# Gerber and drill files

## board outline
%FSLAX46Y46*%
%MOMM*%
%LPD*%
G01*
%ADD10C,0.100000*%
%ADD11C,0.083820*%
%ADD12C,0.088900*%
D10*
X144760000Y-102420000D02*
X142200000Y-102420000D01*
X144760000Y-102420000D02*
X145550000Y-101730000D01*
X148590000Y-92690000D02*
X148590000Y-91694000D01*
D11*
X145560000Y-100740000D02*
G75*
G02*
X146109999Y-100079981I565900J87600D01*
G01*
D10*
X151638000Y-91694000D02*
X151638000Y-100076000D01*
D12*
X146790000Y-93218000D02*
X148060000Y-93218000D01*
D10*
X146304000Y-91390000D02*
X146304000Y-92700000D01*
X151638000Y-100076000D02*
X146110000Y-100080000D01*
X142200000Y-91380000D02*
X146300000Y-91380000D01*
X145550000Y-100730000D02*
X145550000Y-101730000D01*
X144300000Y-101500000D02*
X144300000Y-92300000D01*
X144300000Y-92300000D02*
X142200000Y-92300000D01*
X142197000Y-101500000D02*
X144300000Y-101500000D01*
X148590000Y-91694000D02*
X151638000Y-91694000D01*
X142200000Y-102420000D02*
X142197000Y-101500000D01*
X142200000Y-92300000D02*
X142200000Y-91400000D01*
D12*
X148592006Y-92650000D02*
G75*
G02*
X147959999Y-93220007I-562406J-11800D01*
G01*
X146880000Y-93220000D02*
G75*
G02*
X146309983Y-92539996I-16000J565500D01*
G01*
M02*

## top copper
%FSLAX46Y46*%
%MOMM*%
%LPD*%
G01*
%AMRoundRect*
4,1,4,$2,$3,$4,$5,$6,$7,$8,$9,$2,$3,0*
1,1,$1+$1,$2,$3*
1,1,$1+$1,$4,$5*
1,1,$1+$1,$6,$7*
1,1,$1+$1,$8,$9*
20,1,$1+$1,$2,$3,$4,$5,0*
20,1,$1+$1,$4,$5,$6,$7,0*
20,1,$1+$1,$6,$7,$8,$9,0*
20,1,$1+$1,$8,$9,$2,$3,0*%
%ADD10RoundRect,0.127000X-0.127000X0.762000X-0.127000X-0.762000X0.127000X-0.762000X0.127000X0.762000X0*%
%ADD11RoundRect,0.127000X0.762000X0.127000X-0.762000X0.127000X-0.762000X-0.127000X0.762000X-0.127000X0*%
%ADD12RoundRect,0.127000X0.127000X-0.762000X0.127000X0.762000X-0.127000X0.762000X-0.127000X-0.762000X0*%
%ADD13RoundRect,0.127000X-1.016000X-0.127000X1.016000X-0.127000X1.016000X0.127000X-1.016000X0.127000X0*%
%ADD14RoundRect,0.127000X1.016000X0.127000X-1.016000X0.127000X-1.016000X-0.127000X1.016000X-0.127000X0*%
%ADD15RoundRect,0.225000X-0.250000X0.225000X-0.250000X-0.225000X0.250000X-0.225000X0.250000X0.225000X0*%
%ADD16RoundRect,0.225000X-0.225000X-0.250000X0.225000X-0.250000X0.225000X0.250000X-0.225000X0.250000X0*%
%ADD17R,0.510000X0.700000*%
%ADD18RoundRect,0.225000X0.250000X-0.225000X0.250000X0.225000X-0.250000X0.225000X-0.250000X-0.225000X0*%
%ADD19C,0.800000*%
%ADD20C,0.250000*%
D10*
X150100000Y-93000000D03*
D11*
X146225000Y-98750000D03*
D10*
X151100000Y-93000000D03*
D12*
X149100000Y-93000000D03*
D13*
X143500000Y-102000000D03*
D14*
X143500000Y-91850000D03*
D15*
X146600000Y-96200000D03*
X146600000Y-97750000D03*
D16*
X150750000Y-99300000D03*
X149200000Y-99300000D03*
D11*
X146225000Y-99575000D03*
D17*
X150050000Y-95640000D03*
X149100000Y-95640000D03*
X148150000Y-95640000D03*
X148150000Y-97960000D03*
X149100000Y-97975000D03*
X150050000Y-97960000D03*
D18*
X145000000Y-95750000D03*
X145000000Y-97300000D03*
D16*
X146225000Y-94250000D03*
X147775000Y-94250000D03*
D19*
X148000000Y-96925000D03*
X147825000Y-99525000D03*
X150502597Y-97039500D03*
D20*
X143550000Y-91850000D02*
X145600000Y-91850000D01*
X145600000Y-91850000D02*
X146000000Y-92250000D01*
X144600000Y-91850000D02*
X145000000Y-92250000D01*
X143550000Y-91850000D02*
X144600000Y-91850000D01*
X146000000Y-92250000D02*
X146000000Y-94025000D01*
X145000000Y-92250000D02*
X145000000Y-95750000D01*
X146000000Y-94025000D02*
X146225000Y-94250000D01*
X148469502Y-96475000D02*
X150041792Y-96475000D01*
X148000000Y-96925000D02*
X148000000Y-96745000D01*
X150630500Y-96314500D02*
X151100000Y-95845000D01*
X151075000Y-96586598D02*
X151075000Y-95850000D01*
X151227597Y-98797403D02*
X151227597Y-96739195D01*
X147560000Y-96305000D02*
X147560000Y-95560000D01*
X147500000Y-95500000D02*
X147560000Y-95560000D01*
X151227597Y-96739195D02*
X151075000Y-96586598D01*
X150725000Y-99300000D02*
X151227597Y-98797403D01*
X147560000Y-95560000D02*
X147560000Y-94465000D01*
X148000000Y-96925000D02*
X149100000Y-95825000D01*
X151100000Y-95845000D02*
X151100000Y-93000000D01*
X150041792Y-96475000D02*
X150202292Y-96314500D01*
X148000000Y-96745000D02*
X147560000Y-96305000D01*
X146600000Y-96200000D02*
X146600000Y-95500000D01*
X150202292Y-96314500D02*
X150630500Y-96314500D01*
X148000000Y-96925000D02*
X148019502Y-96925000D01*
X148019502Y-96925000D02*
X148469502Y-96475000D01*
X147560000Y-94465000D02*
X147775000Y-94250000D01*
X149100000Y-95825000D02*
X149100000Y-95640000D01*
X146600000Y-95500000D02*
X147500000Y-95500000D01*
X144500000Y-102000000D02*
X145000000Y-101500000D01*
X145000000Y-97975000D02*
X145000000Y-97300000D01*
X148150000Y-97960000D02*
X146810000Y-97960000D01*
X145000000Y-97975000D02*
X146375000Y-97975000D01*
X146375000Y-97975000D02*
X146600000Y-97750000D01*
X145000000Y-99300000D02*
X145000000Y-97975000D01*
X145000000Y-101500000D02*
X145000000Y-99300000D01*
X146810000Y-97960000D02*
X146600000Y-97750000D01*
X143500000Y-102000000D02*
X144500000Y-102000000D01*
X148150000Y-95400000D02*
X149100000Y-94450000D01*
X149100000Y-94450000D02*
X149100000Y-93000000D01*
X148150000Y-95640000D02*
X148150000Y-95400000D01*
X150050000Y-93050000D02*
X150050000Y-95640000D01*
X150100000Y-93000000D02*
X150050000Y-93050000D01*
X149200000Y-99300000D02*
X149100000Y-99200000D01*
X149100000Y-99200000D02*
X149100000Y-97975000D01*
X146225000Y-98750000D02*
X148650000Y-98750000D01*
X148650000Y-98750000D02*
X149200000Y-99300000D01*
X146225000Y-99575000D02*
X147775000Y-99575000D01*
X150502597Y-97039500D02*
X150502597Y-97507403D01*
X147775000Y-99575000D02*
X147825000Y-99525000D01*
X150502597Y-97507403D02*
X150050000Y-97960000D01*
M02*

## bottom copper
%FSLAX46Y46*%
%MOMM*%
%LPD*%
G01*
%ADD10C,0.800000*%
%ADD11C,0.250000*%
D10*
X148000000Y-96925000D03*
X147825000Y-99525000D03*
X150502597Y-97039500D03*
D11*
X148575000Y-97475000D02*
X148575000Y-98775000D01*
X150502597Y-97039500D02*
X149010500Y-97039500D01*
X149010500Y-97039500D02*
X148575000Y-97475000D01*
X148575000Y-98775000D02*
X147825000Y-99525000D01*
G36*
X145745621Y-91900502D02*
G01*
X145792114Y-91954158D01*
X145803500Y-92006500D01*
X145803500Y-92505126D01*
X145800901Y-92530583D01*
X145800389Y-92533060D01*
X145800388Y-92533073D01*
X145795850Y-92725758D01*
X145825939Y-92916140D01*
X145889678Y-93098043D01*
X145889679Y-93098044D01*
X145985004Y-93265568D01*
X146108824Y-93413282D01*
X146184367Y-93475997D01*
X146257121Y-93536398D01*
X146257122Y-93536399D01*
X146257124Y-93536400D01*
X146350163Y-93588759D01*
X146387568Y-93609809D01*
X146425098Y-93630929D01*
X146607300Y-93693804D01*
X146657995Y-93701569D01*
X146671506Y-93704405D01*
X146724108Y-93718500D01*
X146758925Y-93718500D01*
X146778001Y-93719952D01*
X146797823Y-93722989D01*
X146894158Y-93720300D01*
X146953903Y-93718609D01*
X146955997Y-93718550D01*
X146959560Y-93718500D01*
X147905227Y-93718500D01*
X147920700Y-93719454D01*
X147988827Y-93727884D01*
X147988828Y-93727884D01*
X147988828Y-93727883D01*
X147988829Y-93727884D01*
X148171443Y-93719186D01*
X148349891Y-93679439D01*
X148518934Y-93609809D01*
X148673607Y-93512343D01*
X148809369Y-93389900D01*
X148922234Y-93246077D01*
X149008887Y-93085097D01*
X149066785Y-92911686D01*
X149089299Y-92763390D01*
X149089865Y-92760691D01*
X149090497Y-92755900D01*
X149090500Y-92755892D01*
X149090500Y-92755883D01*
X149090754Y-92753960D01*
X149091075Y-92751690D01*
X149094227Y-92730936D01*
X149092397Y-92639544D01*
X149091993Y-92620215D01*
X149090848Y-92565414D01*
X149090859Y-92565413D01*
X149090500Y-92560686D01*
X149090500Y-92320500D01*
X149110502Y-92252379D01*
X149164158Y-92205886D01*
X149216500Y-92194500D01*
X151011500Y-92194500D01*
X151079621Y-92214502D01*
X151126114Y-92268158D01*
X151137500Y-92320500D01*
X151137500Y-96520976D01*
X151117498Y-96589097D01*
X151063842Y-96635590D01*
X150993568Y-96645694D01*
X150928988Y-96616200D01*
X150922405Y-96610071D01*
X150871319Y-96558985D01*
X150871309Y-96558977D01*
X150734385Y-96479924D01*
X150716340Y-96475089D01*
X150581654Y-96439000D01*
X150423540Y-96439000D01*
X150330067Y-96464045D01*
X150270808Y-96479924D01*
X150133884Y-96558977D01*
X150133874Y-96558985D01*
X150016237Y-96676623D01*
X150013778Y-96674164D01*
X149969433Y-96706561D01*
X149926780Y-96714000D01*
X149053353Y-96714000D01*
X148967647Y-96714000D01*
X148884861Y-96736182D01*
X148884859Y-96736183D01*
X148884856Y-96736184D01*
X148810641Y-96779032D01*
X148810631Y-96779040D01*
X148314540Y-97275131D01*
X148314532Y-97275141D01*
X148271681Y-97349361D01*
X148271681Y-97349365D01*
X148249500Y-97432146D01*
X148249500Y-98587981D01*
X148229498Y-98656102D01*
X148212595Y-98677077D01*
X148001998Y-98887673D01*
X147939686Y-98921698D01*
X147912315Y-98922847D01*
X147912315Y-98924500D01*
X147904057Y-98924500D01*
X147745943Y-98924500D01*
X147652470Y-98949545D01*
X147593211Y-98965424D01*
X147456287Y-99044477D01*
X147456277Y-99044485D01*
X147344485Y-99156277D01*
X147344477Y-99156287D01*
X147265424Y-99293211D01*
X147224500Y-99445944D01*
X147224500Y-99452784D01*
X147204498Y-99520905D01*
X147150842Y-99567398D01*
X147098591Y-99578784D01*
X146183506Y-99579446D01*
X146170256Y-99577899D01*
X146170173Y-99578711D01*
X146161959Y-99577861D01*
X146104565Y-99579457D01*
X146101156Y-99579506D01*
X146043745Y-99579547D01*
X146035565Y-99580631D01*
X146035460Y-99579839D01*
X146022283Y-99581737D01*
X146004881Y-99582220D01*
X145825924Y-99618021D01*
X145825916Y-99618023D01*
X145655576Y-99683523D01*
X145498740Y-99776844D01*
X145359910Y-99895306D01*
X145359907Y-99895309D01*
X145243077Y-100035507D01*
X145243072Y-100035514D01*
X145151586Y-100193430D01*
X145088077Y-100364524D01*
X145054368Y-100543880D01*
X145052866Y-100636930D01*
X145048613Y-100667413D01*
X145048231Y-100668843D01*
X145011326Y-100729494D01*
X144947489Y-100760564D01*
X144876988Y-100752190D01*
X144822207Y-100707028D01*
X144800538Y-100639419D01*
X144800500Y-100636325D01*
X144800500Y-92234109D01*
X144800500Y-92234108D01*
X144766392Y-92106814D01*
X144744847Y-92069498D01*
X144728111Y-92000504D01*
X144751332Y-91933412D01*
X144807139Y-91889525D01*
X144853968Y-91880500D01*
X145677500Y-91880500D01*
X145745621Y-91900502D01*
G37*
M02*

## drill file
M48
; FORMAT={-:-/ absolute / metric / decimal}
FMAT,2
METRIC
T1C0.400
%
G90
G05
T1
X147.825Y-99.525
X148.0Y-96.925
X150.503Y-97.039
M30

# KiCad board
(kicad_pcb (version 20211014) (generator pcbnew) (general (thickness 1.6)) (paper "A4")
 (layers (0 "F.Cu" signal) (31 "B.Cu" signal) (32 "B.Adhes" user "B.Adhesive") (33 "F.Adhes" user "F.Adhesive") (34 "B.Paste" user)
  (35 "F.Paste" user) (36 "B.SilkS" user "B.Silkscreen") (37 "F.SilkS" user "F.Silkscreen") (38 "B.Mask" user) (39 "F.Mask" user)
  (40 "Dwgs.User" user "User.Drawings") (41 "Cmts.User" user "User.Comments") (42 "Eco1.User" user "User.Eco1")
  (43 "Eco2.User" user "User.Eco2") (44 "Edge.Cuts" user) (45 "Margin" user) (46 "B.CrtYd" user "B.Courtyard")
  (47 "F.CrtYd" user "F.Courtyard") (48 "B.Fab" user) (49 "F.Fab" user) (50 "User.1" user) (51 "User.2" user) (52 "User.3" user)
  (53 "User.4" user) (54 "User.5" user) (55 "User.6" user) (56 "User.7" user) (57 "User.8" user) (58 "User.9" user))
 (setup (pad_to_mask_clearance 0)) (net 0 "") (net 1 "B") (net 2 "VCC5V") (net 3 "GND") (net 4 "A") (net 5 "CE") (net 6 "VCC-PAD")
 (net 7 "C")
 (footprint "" (layer "F.Cu") (at 150.1 93 90)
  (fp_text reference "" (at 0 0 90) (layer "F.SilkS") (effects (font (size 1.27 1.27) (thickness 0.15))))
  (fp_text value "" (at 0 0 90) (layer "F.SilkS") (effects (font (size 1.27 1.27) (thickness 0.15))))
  (pad "10" smd roundrect (at 0 0 270) (size 1.778 0.508) (layers "F.Cu" "F.Paste" "F.Mask") (roundrect_rratio 0.25) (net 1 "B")))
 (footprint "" (layer "F.Cu") (at 146.225 98.75 -90)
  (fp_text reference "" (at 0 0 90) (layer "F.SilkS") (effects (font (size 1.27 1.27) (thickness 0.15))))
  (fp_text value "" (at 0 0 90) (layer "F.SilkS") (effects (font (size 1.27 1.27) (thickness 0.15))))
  (pad "B" smd roundrect (at 0 0 180) (size 1.778 0.508) (layers "F.Cu" "F.Paste" "F.Mask") (roundrect_rratio 0.25) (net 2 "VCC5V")))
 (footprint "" (layer "F.Cu") (at 151.1 93 90)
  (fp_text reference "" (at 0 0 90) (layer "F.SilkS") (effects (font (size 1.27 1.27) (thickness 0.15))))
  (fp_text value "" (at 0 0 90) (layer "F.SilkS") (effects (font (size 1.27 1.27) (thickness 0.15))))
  (pad "9" smd roundrect (at 0 0 270) (size 1.778 0.508) (layers "F.Cu" "F.Paste" "F.Mask") (roundrect_rratio 0.25) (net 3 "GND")))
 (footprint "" (layer "F.Cu") (at 149.1 93 -90)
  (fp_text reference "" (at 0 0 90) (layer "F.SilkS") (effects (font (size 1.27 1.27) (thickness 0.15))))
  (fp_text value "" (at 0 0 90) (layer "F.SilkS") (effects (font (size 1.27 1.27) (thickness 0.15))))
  (pad "11" smd roundrect (at 0 0 90) (size 1.778 0.508) (layers "F.Cu" "F.Paste" "F.Mask") (roundrect_rratio 0.25) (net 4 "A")))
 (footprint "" (layer "F.Cu") (at 143.5 102)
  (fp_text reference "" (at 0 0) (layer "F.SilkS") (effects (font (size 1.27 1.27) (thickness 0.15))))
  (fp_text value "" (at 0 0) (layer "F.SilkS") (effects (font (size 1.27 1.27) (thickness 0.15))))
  (pad "4" smd roundrect (at 0 0) (size 2.286 0.508) (layers "F.Cu" "F.Paste" "F.Mask") (roundrect_rratio 0.25) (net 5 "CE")))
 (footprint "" (layer "F.Cu") (at 143.5 91.85 180)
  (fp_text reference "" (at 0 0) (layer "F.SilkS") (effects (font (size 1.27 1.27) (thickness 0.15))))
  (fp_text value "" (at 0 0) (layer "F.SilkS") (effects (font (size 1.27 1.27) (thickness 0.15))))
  (pad "1" smd roundrect (at 0 0 180) (size 2.286 0.508) (layers "F.Cu" "F.Paste" "F.Mask") (roundrect_rratio 0.25) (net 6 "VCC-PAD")))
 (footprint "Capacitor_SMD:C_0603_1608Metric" (layer "F.Cu") (at 146.6 96.975 -90)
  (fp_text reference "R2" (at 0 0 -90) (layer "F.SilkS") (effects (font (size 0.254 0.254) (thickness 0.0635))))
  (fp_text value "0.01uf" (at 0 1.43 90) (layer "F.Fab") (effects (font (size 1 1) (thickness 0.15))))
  (pad "5" smd roundrect (at -0.775 0 270) (size 0.9 0.95) (layers "F.Cu" "F.Paste" "F.Mask") (roundrect_rratio 0.25) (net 3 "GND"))
  (pad "6" smd roundrect (at 0.775 0 270) (size 0.9 0.95) (layers "F.Cu" "F.Paste" "F.Mask") (roundrect_rratio 0.25) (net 5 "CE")))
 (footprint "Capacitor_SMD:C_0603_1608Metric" (layer "F.Cu") (at 149.975 99.3)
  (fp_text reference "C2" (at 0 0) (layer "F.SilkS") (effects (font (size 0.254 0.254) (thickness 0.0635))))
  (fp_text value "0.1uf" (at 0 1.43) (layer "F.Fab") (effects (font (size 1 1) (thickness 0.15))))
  (pad "7" smd roundrect (at 0.775 0) (size 0.9 0.95) (layers "F.Cu" "F.Paste" "F.Mask") (roundrect_rratio 0.25) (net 3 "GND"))
  (pad "8" smd roundrect (at -0.775 0) (size 0.9 0.95) (layers "F.Cu" "F.Paste" "F.Mask") (roundrect_rratio 0.25) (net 2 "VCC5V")))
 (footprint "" (layer "F.Cu") (at 146.225 99.575)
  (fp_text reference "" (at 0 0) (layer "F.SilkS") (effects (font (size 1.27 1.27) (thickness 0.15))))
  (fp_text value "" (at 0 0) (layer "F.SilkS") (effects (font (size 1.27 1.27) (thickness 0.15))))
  (pad "B" smd roundrect (at 0 0 180) (size 1.778 0.508) (layers "F.Cu" "F.Paste" "F.Mask") (roundrect_rratio 0.25) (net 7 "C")))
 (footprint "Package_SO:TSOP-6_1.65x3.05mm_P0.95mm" (layer "F.Cu") (at 149.1 96.8 -90)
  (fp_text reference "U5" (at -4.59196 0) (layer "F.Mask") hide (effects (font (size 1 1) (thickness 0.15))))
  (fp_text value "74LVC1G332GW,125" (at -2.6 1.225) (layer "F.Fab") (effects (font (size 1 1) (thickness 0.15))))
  (pad "1" smd rect (at -1.16 -0.95 270) (size 0.7 0.51) (layers "F.Cu" "F.Paste" "F.Mask") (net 1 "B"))
  (pad "2" smd rect (at -1.16 0 270) (size 0.7 0.51) (layers "F.Cu" "F.Paste" "F.Mask") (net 3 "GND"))
  (pad "3" smd rect (at -1.16 0.95 270) (size 0.7 0.51) (layers "F.Cu" "F.Paste" "F.Mask") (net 4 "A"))
  (pad "4" smd rect (at 1.16 0.95 270) (size 0.7 0.51) (layers "F.Cu" "F.Paste" "F.Mask") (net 5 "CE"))
  (pad "5" smd rect (at 1.175 0 270) (size 0.7 0.51) (layers "F.Cu" "F.Paste" "F.Mask") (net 2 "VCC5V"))
  (pad "6" smd rect (at 1.16 -0.95 270) (size 0.7 0.51) (layers "F.Cu" "F.Paste" "F.Mask") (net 7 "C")))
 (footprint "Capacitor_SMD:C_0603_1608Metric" (layer "F.Cu") (at 145 96.525 90)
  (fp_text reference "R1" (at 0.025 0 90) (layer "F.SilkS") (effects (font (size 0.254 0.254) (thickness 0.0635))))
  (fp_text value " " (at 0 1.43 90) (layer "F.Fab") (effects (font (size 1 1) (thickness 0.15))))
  (pad "2" smd roundrect (at 0.775 0 90) (size 0.9 0.95) (layers "F.Cu" "F.Paste" "F.Mask") (roundrect_rratio 0.25) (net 6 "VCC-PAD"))
  (pad "3" smd roundrect (at -0.775 0 90) (size 0.9 0.95) (layers "F.Cu" "F.Paste" "F.Mask") (roundrect_rratio 0.25) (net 5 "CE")))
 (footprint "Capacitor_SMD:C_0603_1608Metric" (layer "F.Cu") (at 147 94.25)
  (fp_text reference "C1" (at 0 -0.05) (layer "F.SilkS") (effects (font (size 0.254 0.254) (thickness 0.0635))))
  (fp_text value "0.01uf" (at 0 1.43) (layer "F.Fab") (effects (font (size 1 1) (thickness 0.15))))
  (pad "5" smd roundrect (at -0.775 0) (size 0.9 0.95) (layers "F.Cu" "F.Paste" "F.Mask") (roundrect_rratio 0.25) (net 6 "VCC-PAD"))
  (pad "6" smd roundrect (at 0.775 0) (size 0.9 0.95) (layers "F.Cu" "F.Paste" "F.Mask") (roundrect_rratio 0.25) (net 3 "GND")))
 (gr_line (start 144.76 102.42) (end 142.2 102.42) (layer "Edge.Cuts") (width 0.1))
 (gr_line (start 144.76 102.42) (end 145.55 101.73) (layer "Edge.Cuts") (width 0.1))
 (gr_line (start 148.59 92.69) (end 148.59 91.694) (layer "Edge.Cuts") (width 0.1))
 (gr_arc (start 145.56 100.74) (mid 145.684497 100.28762) (end 146.11 100.08) (layer "Edge.Cuts") (width 0.08382))
 (gr_line (start 151.638 91.694) (end 151.638 100.076) (layer "Edge.Cuts") (width 0.1))
 (gr_line (start 146.79 93.218) (end 148.06 93.218) (layer "Edge.Cuts") (width 0.0889))
 (gr_line (start 146.304 91.39) (end 146.304 92.7) (layer "Edge.Cuts") (width 0.1))
 (gr_line (start 151.638 100.076) (end 146.11 100.08) (layer "Edge.Cuts") (width 0.1))
 (gr_line (start 142.2 91.38) (end 146.3 91.38) (layer "Edge.Cuts") (width 0.1))
 (gr_line (start 145.55 100.73) (end 145.55 101.73) (layer "Edge.Cuts") (width 0.1))
 (gr_line (start 144.3 101.5) (end 144.3 92.3) (layer "Edge.Cuts") (width 0.1))
 (gr_line (start 144.3 92.3) (end 142.2 92.3) (layer "Edge.Cuts") (width 0.1))
 (gr_line (start 142.197 101.5) (end 144.3 101.5) (layer "Edge.Cuts") (width 0.1))
 (gr_line (start 148.59 91.694) (end 151.638 91.694) (layer "Edge.Cuts") (width 0.1))
 (gr_line (start 142.2 102.42) (end 142.197 101.5) (layer "Edge.Cuts") (width 0.1))
 (gr_line (start 142.2 92.3) (end 142.2 91.4) (layer "Edge.Cuts") (width 0.1))
 (gr_arc (start 148.592006 92.65) (mid 148.406336 93.079511) (end 147.96 93.22) (layer "Edge.Cuts") (width 0.0889))
 (gr_arc (start 146.88 93.22) (mid 146.430454 93.017928) (end 146.31 92.54) (layer "Edge.Cuts") (width 0.0889))
 (segment (start 143.55 91.85) (end 145.6 91.85) (width 0.25) (layer "F.Cu") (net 6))
 (segment (start 145.6 91.85) (end 146 92.25) (width 0.25) (layer "F.Cu") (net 6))
 (segment (start 144.6 91.85) (end 145 92.25) (width 0.25) (layer "F.Cu") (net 6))
 (segment (start 143.55 91.85) (end 144.6 91.85) (width 0.25) (layer "F.Cu") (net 6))
 (segment (start 146 92.25) (end 146 94.025) (width 0.25) (layer "F.Cu") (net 6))
 (segment (start 145 92.25) (end 145 95.75) (width 0.25) (layer "F.Cu") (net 6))
 (segment (start 146 94.025) (end 146.225 94.25) (width 0.25) (layer "F.Cu") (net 6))
 (segment (start 148.469502 96.475) (end 150.041792 96.475) (width 0.25) (layer "F.Cu") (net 3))
 (segment (start 148 96.925) (end 148 96.745) (width 0.25) (layer "F.Cu") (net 3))
 (segment (start 150.6305 96.3145) (end 151.1 95.845) (width 0.25) (layer "F.Cu") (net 3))
 (segment (start 151.075 96.586598) (end 151.075 95.85) (width 0.25) (layer "F.Cu") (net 3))
 (segment (start 151.227597 98.797403) (end 151.227597 96.739195) (width 0.25) (layer "F.Cu") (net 3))
 (segment (start 147.56 96.305) (end 147.56 95.56) (width 0.25) (layer "F.Cu") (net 3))
 (segment (start 147.5 95.5) (end 147.56 95.56) (width 0.25) (layer "F.Cu") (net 3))
 (segment (start 151.227597 96.739195) (end 151.075 96.586598) (width 0.25) (layer "F.Cu") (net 3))
 (segment (start 150.725 99.3) (end 151.227597 98.797403) (width 0.25) (layer "F.Cu") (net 3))
 (segment (start 147.56 95.56) (end 147.56 94.465) (width 0.25) (layer "F.Cu") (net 3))
 (segment (start 148 96.925) (end 149.1 95.825) (width 0.25) (layer "F.Cu") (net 3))
 (segment (start 151.1 95.845) (end 151.1 93) (width 0.25) (layer "F.Cu") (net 3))
 (segment (start 150.041792 96.475) (end 150.202292 96.3145) (width 0.25) (layer "F.Cu") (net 3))
 (segment (start 148 96.745) (end 147.56 96.305) (width 0.25) (layer "F.Cu") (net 3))
 (segment (start 146.6 96.2) (end 146.6 95.5) (width 0.25) (layer "F.Cu") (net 3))
 (segment (start 150.202292 96.3145) (end 150.6305 96.3145) (width 0.25) (layer "F.Cu") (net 3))
 (segment (start 148 96.925) (end 148.019502 96.925) (width 0.25) (layer "F.Cu") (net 3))
 (segment (start 148.019502 96.925) (end 148.469502 96.475) (width 0.25) (layer "F.Cu") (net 3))
 (segment (start 147.56 94.465) (end 147.775 94.25) (width 0.25) (layer "F.Cu") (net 3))
 (segment (start 149.1 95.825) (end 149.1 95.64) (width 0.25) (layer "F.Cu") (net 3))
 (segment (start 146.6 95.5) (end 147.5 95.5) (width 0.25) (layer "F.Cu") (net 3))
 (via (at 148 96.925) (size 0.8) (drill 0.4) (layers "F.Cu" "B.Cu") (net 3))
 (segment (start 144.5 102) (end 145 101.5) (width 0.25) (layer "F.Cu") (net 5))
 (segment (start 145 97.975) (end 145 97.3) (width 0.25) (layer "F.Cu") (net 5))
 (segment (start 148.15 97.96) (end 146.81 97.96) (width 0.25) (layer "F.Cu") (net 5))
 (segment (start 145 97.975) (end 146.375 97.975) (width 0.25) (layer "F.Cu") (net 5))
 (segment (start 146.375 97.975) (end 146.6 97.75) (width 0.25) (layer "F.Cu") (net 5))
 (segment (start 145 99.3) (end 145 97.975) (width 0.25) (layer "F.Cu") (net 5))
 (segment (start 145 101.5) (end 145 99.3) (width 0.25) (layer "F.Cu") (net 5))
 (segment (start 146.81 97.96) (end 146.6 97.75) (width 0.25) (layer "F.Cu") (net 5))
 (segment (start 143.5 102) (end 144.5 102) (width 0.25) (layer "F.Cu") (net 5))
 (segment (start 148.15 95.4) (end 149.1 94.45) (width 0.25) (layer "F.Cu") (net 4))
 (segment (start 149.1 94.45) (end 149.1 93) (width 0.25) (layer "F.Cu") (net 4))
 (segment (start 148.15 95.64) (end 148.15 95.4) (width 0.25) (layer "F.Cu") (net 4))
 (segment (start 150.05 93.05) (end 150.05 95.64) (width 0.25) (layer "F.Cu") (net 1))
 (segment (start 150.1 93) (end 150.05 93.05) (width 0.25) (layer "F.Cu") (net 1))
 (segment (start 149.2 99.3) (end 149.1 99.2) (width 0.25) (layer "F.Cu") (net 2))
 (segment (start 149.1 99.2) (end 149.1 97.975) (width 0.25) (layer "F.Cu") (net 2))
 (segment (start 146.225 98.75) (end 148.65 98.75) (width 0.25) (layer "F.Cu") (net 2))
 (segment (start 148.65 98.75) (end 149.2 99.3) (width 0.25) (layer "F.Cu") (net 2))
 (segment (start 146.225 99.575) (end 147.775 99.575) (width 0.25) (layer "F.Cu") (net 7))
 (segment (start 150.502597 97.0395) (end 150.502597 97.507403) (width 0.25) (layer "F.Cu") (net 7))
 (segment (start 147.775 99.575) (end 147.825 99.525) (width 0.25) (layer "F.Cu") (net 7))
 (segment (start 150.502597 97.507403) (end 150.05 97.96) (width 0.25) (layer "F.Cu") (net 7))
 (via (at 147.825 99.525) (size 0.8) (drill 0.4) (layers "F.Cu" "B.Cu") (free) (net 7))
 (via (at 150.502597 97.0395) (size 0.8) (drill 0.4) (layers "F.Cu" "B.Cu") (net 7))
 (segment (start 148.575 97.475) (end 148.575 98.775) (width 0.25) (layer "B.Cu") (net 7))
 (segment (start 150.502597 97.0395) (end 149.0105 97.0395) (width 0.25) (layer "B.Cu") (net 7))
 (segment (start 149.0105 97.0395) (end 148.575 97.475) (width 0.25) (layer "B.Cu") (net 7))
 (segment (start 148.575 98.775) (end 147.825 99.525) (width 0.25) (layer "B.Cu") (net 7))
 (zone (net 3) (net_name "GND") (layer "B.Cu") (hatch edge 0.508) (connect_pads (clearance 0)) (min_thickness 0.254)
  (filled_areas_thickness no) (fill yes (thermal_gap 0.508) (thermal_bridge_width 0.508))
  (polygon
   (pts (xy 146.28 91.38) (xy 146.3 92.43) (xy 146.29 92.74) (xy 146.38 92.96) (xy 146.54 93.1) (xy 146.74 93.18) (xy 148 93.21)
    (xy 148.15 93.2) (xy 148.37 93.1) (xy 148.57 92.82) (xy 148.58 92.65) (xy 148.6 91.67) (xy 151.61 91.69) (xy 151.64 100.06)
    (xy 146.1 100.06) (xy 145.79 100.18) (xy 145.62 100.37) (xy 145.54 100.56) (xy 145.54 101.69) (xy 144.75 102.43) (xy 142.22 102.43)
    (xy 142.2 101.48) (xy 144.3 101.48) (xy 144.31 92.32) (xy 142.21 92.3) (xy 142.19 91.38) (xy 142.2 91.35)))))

